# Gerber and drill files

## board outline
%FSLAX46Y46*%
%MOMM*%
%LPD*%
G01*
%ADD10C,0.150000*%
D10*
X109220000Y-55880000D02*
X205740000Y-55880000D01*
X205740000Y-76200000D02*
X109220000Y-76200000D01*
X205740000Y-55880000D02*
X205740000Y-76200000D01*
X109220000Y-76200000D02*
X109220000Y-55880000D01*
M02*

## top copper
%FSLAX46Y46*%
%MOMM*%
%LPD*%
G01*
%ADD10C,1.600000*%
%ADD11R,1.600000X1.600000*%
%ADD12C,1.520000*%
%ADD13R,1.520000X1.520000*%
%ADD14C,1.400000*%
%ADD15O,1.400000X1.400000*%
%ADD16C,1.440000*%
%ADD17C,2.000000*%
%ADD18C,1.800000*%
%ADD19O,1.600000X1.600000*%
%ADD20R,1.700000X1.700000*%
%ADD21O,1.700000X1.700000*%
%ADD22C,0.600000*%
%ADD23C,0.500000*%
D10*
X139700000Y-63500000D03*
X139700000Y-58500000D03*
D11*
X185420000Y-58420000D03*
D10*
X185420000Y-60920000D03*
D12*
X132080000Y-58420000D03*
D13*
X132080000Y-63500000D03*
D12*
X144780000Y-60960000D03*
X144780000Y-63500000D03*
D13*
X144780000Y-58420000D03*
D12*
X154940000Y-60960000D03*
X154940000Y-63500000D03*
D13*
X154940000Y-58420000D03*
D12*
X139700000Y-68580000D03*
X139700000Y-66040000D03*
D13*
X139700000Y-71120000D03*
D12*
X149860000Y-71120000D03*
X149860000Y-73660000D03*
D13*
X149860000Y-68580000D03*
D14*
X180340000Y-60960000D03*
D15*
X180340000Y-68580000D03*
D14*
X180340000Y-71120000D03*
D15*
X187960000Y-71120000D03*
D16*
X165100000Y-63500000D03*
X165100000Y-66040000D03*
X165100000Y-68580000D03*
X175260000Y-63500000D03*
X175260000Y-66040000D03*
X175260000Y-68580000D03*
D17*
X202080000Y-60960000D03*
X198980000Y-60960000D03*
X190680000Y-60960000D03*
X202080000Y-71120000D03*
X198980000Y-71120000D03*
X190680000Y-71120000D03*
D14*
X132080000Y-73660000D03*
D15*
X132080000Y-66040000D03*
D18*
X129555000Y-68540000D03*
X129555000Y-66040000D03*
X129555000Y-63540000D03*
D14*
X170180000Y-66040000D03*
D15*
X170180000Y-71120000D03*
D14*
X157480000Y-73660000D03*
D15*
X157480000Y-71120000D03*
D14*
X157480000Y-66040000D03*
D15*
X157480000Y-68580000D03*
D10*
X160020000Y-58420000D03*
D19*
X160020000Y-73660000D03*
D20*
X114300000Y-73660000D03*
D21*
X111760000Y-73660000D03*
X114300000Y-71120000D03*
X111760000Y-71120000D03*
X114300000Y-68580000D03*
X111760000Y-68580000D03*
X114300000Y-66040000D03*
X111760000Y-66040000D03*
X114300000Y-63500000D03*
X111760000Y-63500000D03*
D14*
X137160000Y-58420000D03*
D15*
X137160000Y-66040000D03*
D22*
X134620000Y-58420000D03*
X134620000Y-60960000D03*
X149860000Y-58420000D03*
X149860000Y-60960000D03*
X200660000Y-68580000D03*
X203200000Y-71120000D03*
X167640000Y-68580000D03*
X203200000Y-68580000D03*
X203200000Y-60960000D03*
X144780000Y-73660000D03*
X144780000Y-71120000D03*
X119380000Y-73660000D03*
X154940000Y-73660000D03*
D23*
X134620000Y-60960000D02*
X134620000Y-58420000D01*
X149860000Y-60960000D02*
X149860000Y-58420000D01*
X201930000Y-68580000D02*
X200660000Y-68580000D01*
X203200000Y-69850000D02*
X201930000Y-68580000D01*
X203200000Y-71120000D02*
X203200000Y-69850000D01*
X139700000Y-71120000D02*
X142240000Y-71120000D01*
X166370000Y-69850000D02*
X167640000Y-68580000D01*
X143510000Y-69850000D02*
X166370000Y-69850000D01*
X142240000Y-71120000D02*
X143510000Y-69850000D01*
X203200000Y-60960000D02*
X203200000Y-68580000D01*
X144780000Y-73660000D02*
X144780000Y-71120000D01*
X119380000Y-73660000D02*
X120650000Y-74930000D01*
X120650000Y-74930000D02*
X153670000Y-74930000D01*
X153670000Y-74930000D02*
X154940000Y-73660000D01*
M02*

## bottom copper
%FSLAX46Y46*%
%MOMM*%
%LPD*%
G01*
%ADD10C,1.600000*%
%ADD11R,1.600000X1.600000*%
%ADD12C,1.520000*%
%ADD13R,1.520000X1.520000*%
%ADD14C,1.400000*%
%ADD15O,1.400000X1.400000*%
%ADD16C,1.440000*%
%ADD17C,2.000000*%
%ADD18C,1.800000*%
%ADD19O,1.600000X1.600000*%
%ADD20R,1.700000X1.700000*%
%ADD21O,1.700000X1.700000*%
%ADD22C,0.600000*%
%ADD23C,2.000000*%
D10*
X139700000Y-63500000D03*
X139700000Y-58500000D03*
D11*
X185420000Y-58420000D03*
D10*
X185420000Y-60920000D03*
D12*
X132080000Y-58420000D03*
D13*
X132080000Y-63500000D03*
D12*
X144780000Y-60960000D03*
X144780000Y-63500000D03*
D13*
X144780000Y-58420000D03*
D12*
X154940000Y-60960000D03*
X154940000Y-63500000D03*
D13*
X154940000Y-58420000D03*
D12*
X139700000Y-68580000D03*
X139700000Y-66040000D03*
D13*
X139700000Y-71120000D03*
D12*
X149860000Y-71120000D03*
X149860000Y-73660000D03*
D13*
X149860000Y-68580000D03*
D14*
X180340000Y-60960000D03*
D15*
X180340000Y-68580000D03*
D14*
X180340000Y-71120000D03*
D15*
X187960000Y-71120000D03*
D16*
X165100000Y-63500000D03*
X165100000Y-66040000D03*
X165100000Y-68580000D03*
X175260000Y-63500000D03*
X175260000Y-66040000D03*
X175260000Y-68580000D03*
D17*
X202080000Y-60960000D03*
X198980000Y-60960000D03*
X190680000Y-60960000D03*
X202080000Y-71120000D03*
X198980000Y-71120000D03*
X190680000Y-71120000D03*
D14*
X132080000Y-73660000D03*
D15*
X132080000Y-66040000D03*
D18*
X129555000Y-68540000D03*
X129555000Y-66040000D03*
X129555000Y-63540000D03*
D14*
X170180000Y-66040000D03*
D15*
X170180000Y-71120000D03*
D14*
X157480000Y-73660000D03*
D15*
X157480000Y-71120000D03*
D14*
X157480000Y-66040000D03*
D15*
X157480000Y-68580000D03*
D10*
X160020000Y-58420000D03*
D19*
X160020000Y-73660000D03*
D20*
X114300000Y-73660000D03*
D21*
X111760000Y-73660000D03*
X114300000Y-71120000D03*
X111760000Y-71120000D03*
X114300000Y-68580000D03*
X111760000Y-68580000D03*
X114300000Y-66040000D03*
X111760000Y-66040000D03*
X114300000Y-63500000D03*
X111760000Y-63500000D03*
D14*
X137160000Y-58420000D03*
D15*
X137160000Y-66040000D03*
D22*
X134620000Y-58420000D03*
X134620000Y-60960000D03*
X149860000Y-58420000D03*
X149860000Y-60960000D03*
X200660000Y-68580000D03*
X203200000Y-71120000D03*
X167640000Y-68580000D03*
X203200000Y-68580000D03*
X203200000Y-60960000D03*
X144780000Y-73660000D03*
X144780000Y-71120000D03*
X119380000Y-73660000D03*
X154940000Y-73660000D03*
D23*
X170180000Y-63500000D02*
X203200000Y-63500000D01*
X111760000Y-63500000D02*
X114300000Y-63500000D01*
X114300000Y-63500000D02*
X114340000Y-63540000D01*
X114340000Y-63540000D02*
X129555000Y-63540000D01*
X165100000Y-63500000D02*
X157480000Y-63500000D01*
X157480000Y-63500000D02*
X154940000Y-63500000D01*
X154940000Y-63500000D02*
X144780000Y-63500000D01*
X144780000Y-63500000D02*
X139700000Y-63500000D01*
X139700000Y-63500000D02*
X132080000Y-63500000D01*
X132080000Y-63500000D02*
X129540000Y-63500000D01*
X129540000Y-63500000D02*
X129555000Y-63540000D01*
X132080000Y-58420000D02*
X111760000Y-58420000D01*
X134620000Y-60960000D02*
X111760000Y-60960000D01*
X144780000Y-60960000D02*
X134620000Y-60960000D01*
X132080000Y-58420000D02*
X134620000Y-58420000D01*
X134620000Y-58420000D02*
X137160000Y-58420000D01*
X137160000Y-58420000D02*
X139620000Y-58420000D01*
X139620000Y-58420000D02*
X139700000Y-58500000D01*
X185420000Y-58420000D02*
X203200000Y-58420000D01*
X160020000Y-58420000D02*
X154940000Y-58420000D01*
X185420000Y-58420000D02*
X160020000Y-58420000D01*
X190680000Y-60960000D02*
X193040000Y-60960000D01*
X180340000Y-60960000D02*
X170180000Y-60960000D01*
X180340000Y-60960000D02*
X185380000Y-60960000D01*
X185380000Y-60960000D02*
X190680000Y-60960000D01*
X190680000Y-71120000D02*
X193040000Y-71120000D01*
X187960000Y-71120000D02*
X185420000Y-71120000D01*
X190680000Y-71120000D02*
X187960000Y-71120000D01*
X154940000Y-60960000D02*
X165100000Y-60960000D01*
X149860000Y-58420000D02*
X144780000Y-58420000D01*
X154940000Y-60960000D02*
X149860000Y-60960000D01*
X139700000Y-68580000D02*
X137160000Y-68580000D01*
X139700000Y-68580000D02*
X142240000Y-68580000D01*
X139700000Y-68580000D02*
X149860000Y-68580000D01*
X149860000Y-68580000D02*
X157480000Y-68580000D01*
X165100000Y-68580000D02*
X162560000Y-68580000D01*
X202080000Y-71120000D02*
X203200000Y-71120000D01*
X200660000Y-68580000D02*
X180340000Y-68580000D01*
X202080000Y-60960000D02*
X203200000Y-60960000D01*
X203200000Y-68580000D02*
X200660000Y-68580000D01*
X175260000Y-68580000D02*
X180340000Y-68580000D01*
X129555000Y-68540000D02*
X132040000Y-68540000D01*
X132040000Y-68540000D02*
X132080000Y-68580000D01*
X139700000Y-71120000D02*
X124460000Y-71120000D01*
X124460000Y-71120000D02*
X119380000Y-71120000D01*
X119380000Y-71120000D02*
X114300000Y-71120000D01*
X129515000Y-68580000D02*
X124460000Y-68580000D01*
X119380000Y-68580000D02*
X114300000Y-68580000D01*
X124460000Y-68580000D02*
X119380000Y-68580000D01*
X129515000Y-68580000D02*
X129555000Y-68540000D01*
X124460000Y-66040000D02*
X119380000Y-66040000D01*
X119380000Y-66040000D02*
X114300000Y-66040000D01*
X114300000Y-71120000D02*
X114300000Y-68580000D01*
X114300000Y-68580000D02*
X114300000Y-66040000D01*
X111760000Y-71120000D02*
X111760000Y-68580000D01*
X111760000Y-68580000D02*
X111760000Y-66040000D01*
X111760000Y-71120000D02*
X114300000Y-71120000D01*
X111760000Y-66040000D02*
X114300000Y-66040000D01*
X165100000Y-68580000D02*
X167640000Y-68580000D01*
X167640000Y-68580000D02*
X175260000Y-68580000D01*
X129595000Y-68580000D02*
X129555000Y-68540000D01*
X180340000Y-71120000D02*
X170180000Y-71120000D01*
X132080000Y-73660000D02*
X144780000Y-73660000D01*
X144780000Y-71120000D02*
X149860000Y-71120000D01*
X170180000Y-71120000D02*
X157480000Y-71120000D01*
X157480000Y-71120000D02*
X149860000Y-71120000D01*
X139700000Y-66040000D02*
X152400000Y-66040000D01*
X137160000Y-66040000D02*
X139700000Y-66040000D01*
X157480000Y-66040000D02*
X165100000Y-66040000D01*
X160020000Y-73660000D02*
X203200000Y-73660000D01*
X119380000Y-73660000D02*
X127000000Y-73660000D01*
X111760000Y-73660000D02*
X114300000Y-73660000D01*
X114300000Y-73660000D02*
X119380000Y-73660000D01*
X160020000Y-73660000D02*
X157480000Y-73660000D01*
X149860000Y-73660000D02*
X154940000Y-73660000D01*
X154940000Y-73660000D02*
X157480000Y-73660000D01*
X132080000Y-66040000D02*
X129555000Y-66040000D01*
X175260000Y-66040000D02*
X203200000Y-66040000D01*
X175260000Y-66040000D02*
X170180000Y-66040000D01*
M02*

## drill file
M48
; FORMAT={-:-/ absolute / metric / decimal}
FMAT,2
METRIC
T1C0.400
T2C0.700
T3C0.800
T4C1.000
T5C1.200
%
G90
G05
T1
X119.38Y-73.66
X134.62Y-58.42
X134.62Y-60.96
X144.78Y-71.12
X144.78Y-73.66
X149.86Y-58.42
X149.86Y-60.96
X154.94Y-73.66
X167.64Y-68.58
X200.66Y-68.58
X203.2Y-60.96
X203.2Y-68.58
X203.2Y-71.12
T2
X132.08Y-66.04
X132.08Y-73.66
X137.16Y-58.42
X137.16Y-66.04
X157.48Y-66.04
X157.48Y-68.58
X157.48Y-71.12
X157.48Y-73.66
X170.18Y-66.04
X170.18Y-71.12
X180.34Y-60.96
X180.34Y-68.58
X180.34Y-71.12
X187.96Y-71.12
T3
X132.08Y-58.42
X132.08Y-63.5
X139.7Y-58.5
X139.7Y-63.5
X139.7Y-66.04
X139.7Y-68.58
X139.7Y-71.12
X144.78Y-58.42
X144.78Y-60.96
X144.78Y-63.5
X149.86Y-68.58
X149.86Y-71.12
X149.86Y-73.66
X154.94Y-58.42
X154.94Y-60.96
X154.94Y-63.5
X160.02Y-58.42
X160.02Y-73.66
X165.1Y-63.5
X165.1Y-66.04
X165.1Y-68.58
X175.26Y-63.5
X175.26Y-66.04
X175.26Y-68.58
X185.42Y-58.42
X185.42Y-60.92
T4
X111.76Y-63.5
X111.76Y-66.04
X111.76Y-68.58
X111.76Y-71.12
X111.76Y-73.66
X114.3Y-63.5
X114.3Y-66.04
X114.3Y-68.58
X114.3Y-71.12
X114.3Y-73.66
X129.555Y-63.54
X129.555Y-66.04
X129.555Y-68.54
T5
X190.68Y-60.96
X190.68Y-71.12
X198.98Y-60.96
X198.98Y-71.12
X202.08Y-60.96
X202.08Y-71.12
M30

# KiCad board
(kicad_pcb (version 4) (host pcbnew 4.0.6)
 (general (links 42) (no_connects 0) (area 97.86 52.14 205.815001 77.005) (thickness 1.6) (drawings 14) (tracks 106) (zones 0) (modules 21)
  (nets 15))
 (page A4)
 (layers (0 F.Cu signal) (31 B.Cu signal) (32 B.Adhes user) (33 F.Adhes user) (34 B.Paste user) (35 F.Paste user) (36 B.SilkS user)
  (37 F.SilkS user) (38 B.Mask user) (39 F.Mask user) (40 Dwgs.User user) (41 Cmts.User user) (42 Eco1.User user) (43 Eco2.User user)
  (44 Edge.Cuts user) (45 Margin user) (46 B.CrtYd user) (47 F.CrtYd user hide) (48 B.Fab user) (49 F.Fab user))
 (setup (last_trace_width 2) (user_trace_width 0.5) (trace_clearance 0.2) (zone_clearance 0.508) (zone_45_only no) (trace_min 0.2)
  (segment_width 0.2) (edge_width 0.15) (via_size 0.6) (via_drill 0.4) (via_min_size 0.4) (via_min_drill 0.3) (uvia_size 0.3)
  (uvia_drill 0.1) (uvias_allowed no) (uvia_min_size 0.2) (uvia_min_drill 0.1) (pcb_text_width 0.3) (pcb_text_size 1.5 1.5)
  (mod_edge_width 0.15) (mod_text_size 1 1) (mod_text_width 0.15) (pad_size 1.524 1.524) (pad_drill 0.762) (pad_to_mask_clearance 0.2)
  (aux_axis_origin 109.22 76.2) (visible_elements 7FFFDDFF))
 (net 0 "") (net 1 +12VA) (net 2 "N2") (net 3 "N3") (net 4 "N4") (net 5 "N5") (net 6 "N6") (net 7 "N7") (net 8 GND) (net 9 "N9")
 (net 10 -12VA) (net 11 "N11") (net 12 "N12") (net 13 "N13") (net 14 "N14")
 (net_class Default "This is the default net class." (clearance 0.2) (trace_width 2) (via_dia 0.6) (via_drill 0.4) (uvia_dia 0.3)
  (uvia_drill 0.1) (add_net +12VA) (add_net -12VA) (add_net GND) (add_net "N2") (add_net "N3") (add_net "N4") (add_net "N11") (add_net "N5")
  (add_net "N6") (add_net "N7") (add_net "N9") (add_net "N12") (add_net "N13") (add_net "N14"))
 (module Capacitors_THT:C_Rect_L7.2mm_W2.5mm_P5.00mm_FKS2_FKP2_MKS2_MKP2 (layer F.Cu) (at 139.7 63.5 90)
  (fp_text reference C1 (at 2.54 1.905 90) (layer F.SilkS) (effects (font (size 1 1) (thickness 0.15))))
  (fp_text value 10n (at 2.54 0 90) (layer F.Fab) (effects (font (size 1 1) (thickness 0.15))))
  (pad 1 thru_hole circle (at 0 0 90) (size 1.6 1.6) (drill 0.8) (layers *.Cu *.Mask) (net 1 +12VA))
  (pad 2 thru_hole circle (at 5 0 90) (size 1.6 1.6) (drill 0.8) (layers *.Cu *.Mask) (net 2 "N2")))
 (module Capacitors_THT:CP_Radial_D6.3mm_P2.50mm (layer F.Cu) (at 185.42 58.42 270)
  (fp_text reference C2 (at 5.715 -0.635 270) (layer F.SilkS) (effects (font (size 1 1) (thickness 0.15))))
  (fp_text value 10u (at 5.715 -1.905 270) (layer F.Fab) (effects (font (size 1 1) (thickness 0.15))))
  (pad 1 thru_hole rect (at 0 0 270) (size 1.6 1.6) (drill 0.8) (layers *.Cu *.Mask) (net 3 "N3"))
  (pad 2 thru_hole circle (at 2.5 0 270) (size 1.6 1.6) (drill 0.8) (layers *.Cu *.Mask) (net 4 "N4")))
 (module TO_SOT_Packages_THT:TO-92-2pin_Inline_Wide (layer F.Cu) (at 132.08 63.5 90)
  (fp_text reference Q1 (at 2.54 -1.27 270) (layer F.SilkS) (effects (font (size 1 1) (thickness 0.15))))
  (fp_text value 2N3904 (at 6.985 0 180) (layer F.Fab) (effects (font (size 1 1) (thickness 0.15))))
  (pad 2 thru_hole circle (at 5.08 0 180) (size 1.52 1.52) (drill 0.8) (layers *.Cu *.Mask) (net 2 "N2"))
  (pad 1 thru_hole rect (at 0 0 180) (size 1.52 1.52) (drill 0.8) (layers *.Cu *.Mask) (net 1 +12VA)))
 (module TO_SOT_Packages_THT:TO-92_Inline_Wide (layer F.Cu) (at 144.78 58.42 270)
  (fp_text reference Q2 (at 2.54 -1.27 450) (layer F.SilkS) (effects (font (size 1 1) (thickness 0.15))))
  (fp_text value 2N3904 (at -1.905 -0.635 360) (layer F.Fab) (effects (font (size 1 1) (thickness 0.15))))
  (pad 2 thru_hole circle (at 2.54 0) (size 1.52 1.52) (drill 0.8) (layers *.Cu *.Mask) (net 2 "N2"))
  (pad 3 thru_hole circle (at 5.08 0) (size 1.52 1.52) (drill 0.8) (layers *.Cu *.Mask) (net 1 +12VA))
  (pad 1 thru_hole rect (at 0 0) (size 1.52 1.52) (drill 0.8) (layers *.Cu *.Mask) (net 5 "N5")))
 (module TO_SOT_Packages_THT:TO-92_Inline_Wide (layer F.Cu) (at 154.94 58.42 270)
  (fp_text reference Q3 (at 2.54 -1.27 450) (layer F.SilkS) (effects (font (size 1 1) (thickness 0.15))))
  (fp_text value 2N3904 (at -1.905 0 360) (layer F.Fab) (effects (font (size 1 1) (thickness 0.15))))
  (pad 2 thru_hole circle (at 2.54 0) (size 1.52 1.52) (drill 0.8) (layers *.Cu *.Mask) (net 5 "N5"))
  (pad 3 thru_hole circle (at 5.08 0) (size 1.52 1.52) (drill 0.8) (layers *.Cu *.Mask) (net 1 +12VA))
  (pad 1 thru_hole rect (at 0 0) (size 1.52 1.52) (drill 0.8) (layers *.Cu *.Mask) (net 3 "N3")))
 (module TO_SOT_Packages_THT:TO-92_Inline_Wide (layer F.Cu) (at 139.7 71.12 90)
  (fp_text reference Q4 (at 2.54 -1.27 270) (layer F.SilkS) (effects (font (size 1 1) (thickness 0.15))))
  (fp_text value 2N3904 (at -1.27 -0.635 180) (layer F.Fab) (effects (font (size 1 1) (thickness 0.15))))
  (pad 2 thru_hole circle (at 2.54 0 180) (size 1.52 1.52) (drill 0.8) (layers *.Cu *.Mask) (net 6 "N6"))
  (pad 3 thru_hole circle (at 5.08 0 180) (size 1.52 1.52) (drill 0.8) (layers *.Cu *.Mask) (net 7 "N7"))
  (pad 1 thru_hole rect (at 0 0 180) (size 1.52 1.52) (drill 0.8) (layers *.Cu *.Mask) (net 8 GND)))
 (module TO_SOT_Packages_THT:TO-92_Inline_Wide (layer F.Cu) (at 149.86 68.58 270)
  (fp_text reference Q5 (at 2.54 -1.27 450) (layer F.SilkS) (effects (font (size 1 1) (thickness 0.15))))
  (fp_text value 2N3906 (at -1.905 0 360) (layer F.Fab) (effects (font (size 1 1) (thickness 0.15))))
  (pad 2 thru_hole circle (at 2.54 0) (size 1.52 1.52) (drill 0.8) (layers *.Cu *.Mask) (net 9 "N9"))
  (pad 3 thru_hole circle (at 5.08 0) (size 1.52 1.52) (drill 0.8) (layers *.Cu *.Mask) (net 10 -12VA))
  (pad 1 thru_hole rect (at 0 0) (size 1.52 1.52) (drill 0.8) (layers *.Cu *.Mask) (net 6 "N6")))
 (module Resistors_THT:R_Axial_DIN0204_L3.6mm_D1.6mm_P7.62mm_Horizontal (layer F.Cu) (at 180.34 60.96 270)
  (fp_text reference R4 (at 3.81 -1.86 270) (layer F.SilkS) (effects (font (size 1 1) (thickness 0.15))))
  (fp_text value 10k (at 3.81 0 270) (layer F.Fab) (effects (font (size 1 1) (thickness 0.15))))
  (pad 1 thru_hole circle (at 0 0 270) (size 1.4 1.4) (drill 0.7) (layers *.Cu *.Mask) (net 4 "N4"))
  (pad 2 thru_hole oval (at 7.62 0 270) (size 1.4 1.4) (drill 0.7) (layers *.Cu *.Mask) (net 8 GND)))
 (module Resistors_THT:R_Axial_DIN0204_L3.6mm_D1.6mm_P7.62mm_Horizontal (layer F.Cu) (at 180.34 71.12)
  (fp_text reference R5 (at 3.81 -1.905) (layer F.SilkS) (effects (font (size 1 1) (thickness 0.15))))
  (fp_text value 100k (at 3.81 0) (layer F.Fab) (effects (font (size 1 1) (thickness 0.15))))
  (pad 1 thru_hole circle (at 0 0) (size 1.4 1.4) (drill 0.7) (layers *.Cu *.Mask) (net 9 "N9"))
  (pad 2 thru_hole oval (at 7.62 0) (size 1.4 1.4) (drill 0.7) (layers *.Cu *.Mask) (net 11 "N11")))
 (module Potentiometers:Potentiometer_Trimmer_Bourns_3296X (layer F.Cu) (at 165.1 63.5 90)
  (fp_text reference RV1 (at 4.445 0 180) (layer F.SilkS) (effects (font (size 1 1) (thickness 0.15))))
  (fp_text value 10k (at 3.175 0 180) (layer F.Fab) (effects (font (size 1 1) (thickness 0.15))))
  (pad 1 thru_hole circle (at 0 0 90) (size 1.44 1.44) (drill 0.8) (layers *.Cu *.Mask) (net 1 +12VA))
  (pad 2 thru_hole circle (at -2.54 0 90) (size 1.44 1.44) (drill 0.8) (layers *.Cu *.Mask) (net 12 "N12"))
  (pad 3 thru_hole circle (at -5.08 0 90) (size 1.44 1.44) (drill 0.8) (layers *.Cu *.Mask) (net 8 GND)))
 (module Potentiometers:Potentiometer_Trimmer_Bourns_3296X (layer F.Cu) (at 175.26 63.5 90)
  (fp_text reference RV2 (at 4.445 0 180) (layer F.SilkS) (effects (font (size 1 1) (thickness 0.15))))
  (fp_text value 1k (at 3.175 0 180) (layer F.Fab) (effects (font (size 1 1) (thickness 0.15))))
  (pad 1 thru_hole circle (at 0 0 90) (size 1.44 1.44) (drill 0.8) (layers *.Cu *.Mask))
  (pad 2 thru_hole circle (at -2.54 0 90) (size 1.44 1.44) (drill 0.8) (layers *.Cu *.Mask) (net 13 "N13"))
  (pad 3 thru_hole circle (at -5.08 0 90) (size 1.44 1.44) (drill 0.8) (layers *.Cu *.Mask) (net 8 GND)))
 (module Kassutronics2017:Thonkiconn (layer F.Cu) (at 195.58 60.96 90)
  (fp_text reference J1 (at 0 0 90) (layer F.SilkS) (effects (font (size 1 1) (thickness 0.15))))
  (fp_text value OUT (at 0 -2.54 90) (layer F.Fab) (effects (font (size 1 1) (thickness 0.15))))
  (pad 3 thru_hole circle (at 0 6.5 90) (size 2 2) (drill 1.2) (layers *.Cu *.Mask) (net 8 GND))
  (pad 2 thru_hole circle (at 0 3.4 90) (size 2 2) (drill 1.2) (layers *.Cu *.Mask))
  (pad 1 thru_hole circle (at 0 -4.9 90) (size 2 2) (drill 1.2) (layers *.Cu *.Mask) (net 4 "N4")))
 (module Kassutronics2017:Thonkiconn (layer F.Cu) (at 195.58 71.12 90)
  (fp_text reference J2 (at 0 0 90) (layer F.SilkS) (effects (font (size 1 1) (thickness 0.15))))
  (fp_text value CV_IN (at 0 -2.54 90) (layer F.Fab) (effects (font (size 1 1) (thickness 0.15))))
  (pad 3 thru_hole circle (at 0 6.5 90) (size 2 2) (drill 1.2) (layers *.Cu *.Mask) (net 8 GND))
  (pad 2 thru_hole circle (at 0 3.4 90) (size 2 2) (drill 1.2) (layers *.Cu *.Mask))
  (pad 1 thru_hole circle (at 0 -4.9 90) (size 2 2) (drill 1.2) (layers *.Cu *.Mask) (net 11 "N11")))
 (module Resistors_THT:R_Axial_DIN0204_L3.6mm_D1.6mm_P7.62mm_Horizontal (layer F.Cu) (at 132.08 73.66 90)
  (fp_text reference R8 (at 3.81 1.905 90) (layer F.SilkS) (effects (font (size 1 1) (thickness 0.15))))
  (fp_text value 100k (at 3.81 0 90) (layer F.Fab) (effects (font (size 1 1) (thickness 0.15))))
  (pad 1 thru_hole circle (at 0 0 90) (size 1.4 1.4) (drill 0.7) (layers *.Cu *.Mask) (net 9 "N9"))
  (pad 2 thru_hole oval (at 7.62 0 90) (size 1.4 1.4) (drill 0.7) (layers *.Cu *.Mask) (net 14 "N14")))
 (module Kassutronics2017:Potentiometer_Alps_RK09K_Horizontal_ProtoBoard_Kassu (layer F.Cu) (at 129.54 66.04 180)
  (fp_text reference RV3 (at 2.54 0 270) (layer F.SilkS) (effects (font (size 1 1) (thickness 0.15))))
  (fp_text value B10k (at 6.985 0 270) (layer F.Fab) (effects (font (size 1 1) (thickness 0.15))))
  (pad 3 thru_hole circle (at -0.015 -2.5 180) (size 1.8 1.8) (drill 1) (layers *.Cu *.Mask) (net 8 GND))
  (pad 2 thru_hole circle (at -0.015 0 180) (size 1.8 1.8) (drill 1) (layers *.Cu *.Mask) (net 14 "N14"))
  (pad 1 thru_hole circle (at -0.015 2.5 180) (size 1.8 1.8) (drill 1) (layers *.Cu *.Mask) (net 1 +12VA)))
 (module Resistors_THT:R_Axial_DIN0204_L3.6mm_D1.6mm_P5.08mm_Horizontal (layer F.Cu) (at 170.18 66.04 270)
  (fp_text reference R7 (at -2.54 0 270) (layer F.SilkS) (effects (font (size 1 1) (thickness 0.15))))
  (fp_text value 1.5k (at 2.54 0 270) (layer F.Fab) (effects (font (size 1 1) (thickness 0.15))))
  (pad 1 thru_hole circle (at 0 0 270) (size 1.4 1.4) (drill 0.7) (layers *.Cu *.Mask) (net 13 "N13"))
  (pad 2 thru_hole oval (at 5.08 0 270) (size 1.4 1.4) (drill 0.7) (layers *.Cu *.Mask) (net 9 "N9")))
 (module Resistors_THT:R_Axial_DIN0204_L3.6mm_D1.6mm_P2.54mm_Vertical (layer F.Cu) (at 157.48 73.66 90)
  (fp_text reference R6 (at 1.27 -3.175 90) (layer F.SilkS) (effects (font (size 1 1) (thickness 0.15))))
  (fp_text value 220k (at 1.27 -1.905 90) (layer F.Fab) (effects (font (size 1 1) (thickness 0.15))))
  (pad 1 thru_hole circle (at 0 0 90) (size 1.4 1.4) (drill 0.7) (layers *.Cu *.Mask) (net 10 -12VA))
  (pad 2 thru_hole oval (at 2.54 0 90) (size 1.4 1.4) (drill 0.7) (layers *.Cu *.Mask) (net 9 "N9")))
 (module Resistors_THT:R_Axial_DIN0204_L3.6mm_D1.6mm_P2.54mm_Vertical (layer F.Cu) (at 157.48 66.04 270)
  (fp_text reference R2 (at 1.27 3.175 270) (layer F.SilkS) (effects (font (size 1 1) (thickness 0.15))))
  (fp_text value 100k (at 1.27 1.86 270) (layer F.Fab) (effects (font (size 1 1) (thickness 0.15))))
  (pad 1 thru_hole circle (at 0 0 270) (size 1.4 1.4) (drill 0.7) (layers *.Cu *.Mask) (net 12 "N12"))
  (pad 2 thru_hole oval (at 2.54 0 270) (size 1.4 1.4) (drill 0.7) (layers *.Cu *.Mask) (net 6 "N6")))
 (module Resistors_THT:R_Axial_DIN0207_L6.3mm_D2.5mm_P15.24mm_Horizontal (layer F.Cu) (at 160.02 58.42 270)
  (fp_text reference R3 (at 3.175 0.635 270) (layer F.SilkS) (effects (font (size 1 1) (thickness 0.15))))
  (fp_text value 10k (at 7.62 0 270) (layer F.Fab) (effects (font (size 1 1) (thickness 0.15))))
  (pad 1 thru_hole circle (at 0 0 270) (size 1.6 1.6) (drill 0.8) (layers *.Cu *.Mask) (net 3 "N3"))
  (pad 2 thru_hole oval (at 15.24 0 270) (size 1.6 1.6) (drill 0.8) (layers *.Cu *.Mask) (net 10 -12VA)))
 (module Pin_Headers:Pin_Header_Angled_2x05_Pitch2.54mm (layer F.Cu) (at 114.3 73.66 180)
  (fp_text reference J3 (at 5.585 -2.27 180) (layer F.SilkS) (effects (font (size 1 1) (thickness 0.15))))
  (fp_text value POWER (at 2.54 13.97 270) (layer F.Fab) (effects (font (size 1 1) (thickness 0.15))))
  (pad 1 thru_hole rect (at 0 0 180) (size 1.7 1.7) (drill 1) (layers *.Cu *.Mask) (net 10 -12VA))
  (pad 2 thru_hole oval (at 2.54 0 180) (size 1.7 1.7) (drill 1) (layers *.Cu *.Mask) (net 10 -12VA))
  (pad 3 thru_hole oval (at 0 2.54 180) (size 1.7 1.7) (drill 1) (layers *.Cu *.Mask) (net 8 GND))
  (pad 4 thru_hole oval (at 2.54 2.54 180) (size 1.7 1.7) (drill 1) (layers *.Cu *.Mask) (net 8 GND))
  (pad 5 thru_hole oval (at 0 5.08 180) (size 1.7 1.7) (drill 1) (layers *.Cu *.Mask) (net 8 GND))
  (pad 6 thru_hole oval (at 2.54 5.08 180) (size 1.7 1.7) (drill 1) (layers *.Cu *.Mask) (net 8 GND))
  (pad 7 thru_hole oval (at 0 7.62 180) (size 1.7 1.7) (drill 1) (layers *.Cu *.Mask) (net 8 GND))
  (pad 8 thru_hole oval (at 2.54 7.62 180) (size 1.7 1.7) (drill 1) (layers *.Cu *.Mask) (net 8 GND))
  (pad 9 thru_hole oval (at 0 10.16 180) (size 1.7 1.7) (drill 1) (layers *.Cu *.Mask) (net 1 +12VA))
  (pad 10 thru_hole oval (at 2.54 10.16 180) (size 1.7 1.7) (drill 1) (layers *.Cu *.Mask) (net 1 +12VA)))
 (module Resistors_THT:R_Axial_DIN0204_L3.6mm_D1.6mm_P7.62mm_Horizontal (layer F.Cu) (at 137.16 58.42 270)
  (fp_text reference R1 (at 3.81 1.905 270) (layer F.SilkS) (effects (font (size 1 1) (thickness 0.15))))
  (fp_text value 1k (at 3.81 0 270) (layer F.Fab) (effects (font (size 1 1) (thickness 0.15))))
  (pad 1 thru_hole circle (at 0 0 270) (size 1.4 1.4) (drill 0.7) (layers *.Cu *.Mask) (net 2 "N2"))
  (pad 2 thru_hole oval (at 7.62 0 270) (size 1.4 1.4) (drill 0.7) (layers *.Cu *.Mask) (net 7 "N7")))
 (gr_line (start 109.22 55.88) (end 205.74 55.88) (angle 90) (layer Edge.Cuts) (width 0.15))
 (gr_line (start 205.74 76.2) (end 109.22 76.2) (angle 90) (layer Edge.Cuts) (width 0.15))
 (gr_line (start 205.74 55.88) (end 205.74 76.2) (angle 90) (layer Edge.Cuts) (width 0.15))
 (gr_line (start 109.22 76.2) (end 109.22 55.88) (angle 90) (layer Edge.Cuts) (width 0.15))
 (segment (start 170.18 63.5) (end 203.2 63.5) (width 2) (layer B.Cu) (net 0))
 (segment (start 111.76 63.5) (end 114.3 63.5) (width 2) (layer B.Cu) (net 1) (status 30))
 (segment (start 114.3 63.5) (end 114.34 63.54) (width 2) (layer B.Cu) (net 1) (status 30))
 (segment (start 114.34 63.54) (end 129.555 63.54) (width 2) (layer B.Cu) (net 1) (status 10))
 (segment (start 165.1 63.5) (end 157.48 63.5) (width 2) (layer B.Cu) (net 1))
 (segment (start 157.48 63.5) (end 154.94 63.5) (width 2) (layer B.Cu) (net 1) (status 20))
 (segment (start 154.94 63.5) (end 144.78 63.5) (width 2) (layer B.Cu) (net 1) (status 10))
 (segment (start 144.78 63.5) (end 139.7 63.5) (width 2) (layer B.Cu) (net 1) (status 20))
 (segment (start 139.7 63.5) (end 132.08 63.5) (width 2) (layer B.Cu) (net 1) (status 20))
 (segment (start 132.08 63.5) (end 129.54 63.5) (width 2) (layer B.Cu) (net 1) (status 10))
 (segment (start 129.54 63.5) (end 129.555 63.54) (width 2) (layer B.Cu) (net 1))
 (segment (start 132.08 58.42) (end 111.76 58.42) (width 2) (layer B.Cu) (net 2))
 (segment (start 134.62 60.96) (end 111.76 60.96) (width 2) (layer B.Cu) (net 2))
 (segment (start 144.78 60.96) (end 134.62 60.96) (width 2) (layer B.Cu) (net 2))
 (via (at 134.62 58.42) (size 0.6) (drill 0.4) (layers F.Cu B.Cu) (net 2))
 (segment (start 134.62 60.96) (end 134.62 58.42) (width 0.5) (layer F.Cu) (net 2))
 (via (at 134.62 60.96) (size 0.6) (drill 0.4) (layers F.Cu B.Cu) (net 2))
 (segment (start 132.08 58.42) (end 134.62 58.42) (width 2) (layer B.Cu) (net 2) (status 10))
 (segment (start 134.62 58.42) (end 137.16 58.42) (width 2) (layer B.Cu) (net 2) (status 10))
 (segment (start 137.16 58.42) (end 139.62 58.42) (width 2) (layer B.Cu) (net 2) (status 20))
 (segment (start 139.62 58.42) (end 139.7 58.5) (width 2) (layer B.Cu) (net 2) (status 30))
 (segment (start 185.42 58.42) (end 203.2 58.42) (width 2) (layer B.Cu) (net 3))
 (segment (start 160.02 58.42) (end 154.94 58.42) (width 2) (layer B.Cu) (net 3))
 (segment (start 185.42 58.42) (end 160.02 58.42) (width 2) (layer B.Cu) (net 3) (status 10))
 (segment (start 190.68 60.96) (end 193.04 60.96) (width 2) (layer B.Cu) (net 4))
 (segment (start 180.34 60.96) (end 170.18 60.96) (width 2) (layer B.Cu) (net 4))
 (segment (start 180.34 60.96) (end 185.38 60.96) (width 2) (layer B.Cu) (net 4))
 (segment (start 185.38 60.96) (end 190.68 60.96) (width 2) (layer B.Cu) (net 4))
 (segment (start 190.68 71.12) (end 193.04 71.12) (width 2) (layer B.Cu) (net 11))
 (segment (start 187.96 71.12) (end 185.42 71.12) (width 2) (layer B.Cu) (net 11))
 (segment (start 190.68 71.12) (end 187.96 71.12) (width 2) (layer B.Cu) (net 11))
 (segment (start 154.94 60.96) (end 165.1 60.96) (width 2) (layer B.Cu) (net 5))
 (segment (start 149.86 58.42) (end 144.78 58.42) (width 2) (layer B.Cu) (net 5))
 (via (at 149.86 58.42) (size 0.6) (drill 0.4) (layers F.Cu B.Cu) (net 5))
 (segment (start 149.86 60.96) (end 149.86 58.42) (width 0.5) (layer F.Cu) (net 5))
 (via (at 149.86 60.96) (size 0.6) (drill 0.4) (layers F.Cu B.Cu) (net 5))
 (segment (start 154.94 60.96) (end 149.86 60.96) (width 2) (layer B.Cu) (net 5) (status 10))
 (segment (start 139.7 68.58) (end 137.16 68.58) (width 2) (layer B.Cu) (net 6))
 (segment (start 139.7 68.58) (end 142.24 68.58) (width 2) (layer B.Cu) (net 6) (status 10))
 (segment (start 139.7 68.58) (end 149.86 68.58) (width 2) (layer B.Cu) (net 6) (status 20))
 (segment (start 149.86 68.58) (end 157.48 68.58) (width 2) (layer B.Cu) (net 6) (status 10))
 (segment (start 165.1 68.58) (end 162.56 68.58) (width 2) (layer B.Cu) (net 8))
 (via (at 200.66 68.58) (size 0.6) (drill 0.4) (layers F.Cu B.Cu) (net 8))
 (segment (start 201.93 68.58) (end 200.66 68.58) (width 0.5) (layer F.Cu) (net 8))
 (segment (start 203.2 69.85) (end 201.93 68.58) (width 0.5) (layer F.Cu) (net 8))
 (segment (start 203.2 71.12) (end 203.2 69.85) (width 0.5) (layer F.Cu) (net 8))
 (via (at 203.2 71.12) (size 0.6) (drill 0.4) (layers F.Cu B.Cu) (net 8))
 (segment (start 202.08 71.12) (end 203.2 71.12) (width 2) (layer B.Cu) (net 8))
 (segment (start 200.66 68.58) (end 180.34 68.58) (width 2) (layer B.Cu) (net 8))
 (segment (start 139.7 71.12) (end 142.24 71.12) (width 0.5) (layer F.Cu) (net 8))
 (via (at 167.64 68.58) (size 0.6) (drill 0.4) (layers F.Cu B.Cu) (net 8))
 (segment (start 166.37 69.85) (end 167.64 68.58) (width 0.5) (layer F.Cu) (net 8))
 (segment (start 143.51 69.85) (end 166.37 69.85) (width 0.5) (layer F.Cu) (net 8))
 (segment (start 142.24 71.12) (end 143.51 69.85) (width 0.5) (layer F.Cu) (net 8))
 (segment (start 202.08 60.96) (end 203.2 60.96) (width 2) (layer B.Cu) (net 8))
 (segment (start 203.2 68.58) (end 200.66 68.58) (width 2) (layer B.Cu) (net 8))
 (via (at 203.2 68.58) (size 0.6) (drill 0.4) (layers F.Cu B.Cu) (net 8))
 (segment (start 203.2 60.96) (end 203.2 68.58) (width 0.5) (layer F.Cu) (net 8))
 (via (at 203.2 60.96) (size 0.6) (drill 0.4) (layers F.Cu B.Cu) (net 8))
 (segment (start 175.26 68.58) (end 180.34 68.58) (width 2) (layer B.Cu) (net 8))
 (segment (start 129.555 68.54) (end 132.04 68.54) (width 2) (layer B.Cu) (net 8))
 (segment (start 132.04 68.54) (end 132.08 68.58) (width 2) (layer B.Cu) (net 8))
 (segment (start 139.7 71.12) (end 124.46 71.12) (width 2) (layer B.Cu) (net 8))
 (segment (start 124.46 71.12) (end 119.38 71.12) (width 2) (layer B.Cu) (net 8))
 (segment (start 119.38 71.12) (end 114.3 71.12) (width 2) (layer B.Cu) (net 8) (status 20))
 (segment (start 129.515 68.58) (end 124.46 68.58) (width 2) (layer B.Cu) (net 8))
 (segment (start 119.38 68.58) (end 114.3 68.58) (width 2) (layer B.Cu) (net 8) (status 20))
 (segment (start 124.46 68.58) (end 119.38 68.58) (width 2) (layer B.Cu) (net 8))
 (segment (start 129.515 68.58) (end 129.555 68.54) (width 2) (layer B.Cu) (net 8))
 (segment (start 124.46 66.04) (end 119.38 66.04) (width 2) (layer B.Cu) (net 8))
 (segment (start 119.38 66.04) (end 114.3 66.04) (width 2) (layer B.Cu) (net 8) (status 20))
 (segment (start 114.3 71.12) (end 114.3 68.58) (width 2) (layer B.Cu) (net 8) (status 30))
 (segment (start 114.3 68.58) (end 114.3 66.04) (width 2) (layer B.Cu) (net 8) (status 30))
 (segment (start 111.76 71.12) (end 111.76 68.58) (width 2) (layer B.Cu) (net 8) (status 30))
 (segment (start 111.76 68.58) (end 111.76 66.04) (width 2) (layer B.Cu) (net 8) (status 30))
 (segment (start 111.76 71.12) (end 114.3 71.12) (width 2) (layer B.Cu) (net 8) (status 30))
 (segment (start 111.76 66.04) (end 114.3 66.04) (width 2) (layer B.Cu) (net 8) (status 30))
 (segment (start 165.1 68.58) (end 167.64 68.58) (width 2) (layer B.Cu) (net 8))
 (segment (start 167.64 68.58) (end 175.26 68.58) (width 2) (layer B.Cu) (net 8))
 (segment (start 129.595 68.58) (end 129.555 68.54) (width 2) (layer B.Cu) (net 8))
 (segment (start 180.34 71.12) (end 170.18 71.12) (width 2) (layer B.Cu) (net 9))
 (via (at 144.78 73.66) (size 0.6) (drill 0.4) (layers F.Cu B.Cu) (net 9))
 (segment (start 132.08 73.66) (end 144.78 73.66) (width 2) (layer B.Cu) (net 9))
 (segment (start 144.78 71.12) (end 149.86 71.12) (width 2) (layer B.Cu) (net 9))
 (via (at 144.78 71.12) (size 0.6) (drill 0.4) (layers F.Cu B.Cu) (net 9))
 (segment (start 144.78 73.66) (end 144.78 71.12) (width 0.5) (layer F.Cu) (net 9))
 (segment (start 170.18 71.12) (end 157.48 71.12) (width 2) (layer B.Cu) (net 9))
 (segment (start 157.48 71.12) (end 149.86 71.12) (width 2) (layer B.Cu) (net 9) (status 20))
 (segment (start 139.7 66.04) (end 152.4 66.04) (width 2) (layer B.Cu) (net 7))
 (segment (start 137.16 66.04) (end 139.7 66.04) (width 2) (layer B.Cu) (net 7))
 (segment (start 157.48 66.04) (end 165.1 66.04) (width 2) (layer B.Cu) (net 12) (status 10))
 (segment (start 160.02 73.66) (end 203.2 73.66) (width 2) (layer B.Cu) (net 10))
 (segment (start 119.38 73.66) (end 127 73.66) (width 2) (layer B.Cu) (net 10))
 (segment (start 111.76 73.66) (end 114.3 73.66) (width 2) (layer B.Cu) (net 10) (status 30))
 (segment (start 114.3 73.66) (end 119.38 73.66) (width 2) (layer B.Cu) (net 10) (status 10))
 (via (at 119.38 73.66) (size 0.6) (drill 0.4) (layers F.Cu B.Cu) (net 10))
 (segment (start 119.38 73.66) (end 120.65 74.93) (width 0.5) (layer F.Cu) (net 10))
 (segment (start 120.65 74.93) (end 153.67 74.93) (width 0.5) (layer F.Cu) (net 10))
 (segment (start 153.67 74.93) (end 154.94 73.66) (width 0.5) (layer F.Cu) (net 10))
 (via (at 154.94 73.66) (size 0.6) (drill 0.4) (layers F.Cu B.Cu) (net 10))
 (segment (start 160.02 73.66) (end 157.48 73.66) (width 2) (layer B.Cu) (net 10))
 (segment (start 149.86 73.66) (end 154.94 73.66) (width 2) (layer B.Cu) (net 10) (status 10))
 (segment (start 154.94 73.66) (end 157.48 73.66) (width 2) (layer B.Cu) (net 10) (status 20))
 (segment (start 132.08 66.04) (end 129.555 66.04) (width 2) (layer B.Cu) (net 14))
 (segment (start 175.26 66.04) (end 203.2 66.04) (width 2) (layer B.Cu) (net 13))
 (segment (start 175.26 66.04) (end 170.18 66.04) (width 2) (layer B.Cu) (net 13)))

